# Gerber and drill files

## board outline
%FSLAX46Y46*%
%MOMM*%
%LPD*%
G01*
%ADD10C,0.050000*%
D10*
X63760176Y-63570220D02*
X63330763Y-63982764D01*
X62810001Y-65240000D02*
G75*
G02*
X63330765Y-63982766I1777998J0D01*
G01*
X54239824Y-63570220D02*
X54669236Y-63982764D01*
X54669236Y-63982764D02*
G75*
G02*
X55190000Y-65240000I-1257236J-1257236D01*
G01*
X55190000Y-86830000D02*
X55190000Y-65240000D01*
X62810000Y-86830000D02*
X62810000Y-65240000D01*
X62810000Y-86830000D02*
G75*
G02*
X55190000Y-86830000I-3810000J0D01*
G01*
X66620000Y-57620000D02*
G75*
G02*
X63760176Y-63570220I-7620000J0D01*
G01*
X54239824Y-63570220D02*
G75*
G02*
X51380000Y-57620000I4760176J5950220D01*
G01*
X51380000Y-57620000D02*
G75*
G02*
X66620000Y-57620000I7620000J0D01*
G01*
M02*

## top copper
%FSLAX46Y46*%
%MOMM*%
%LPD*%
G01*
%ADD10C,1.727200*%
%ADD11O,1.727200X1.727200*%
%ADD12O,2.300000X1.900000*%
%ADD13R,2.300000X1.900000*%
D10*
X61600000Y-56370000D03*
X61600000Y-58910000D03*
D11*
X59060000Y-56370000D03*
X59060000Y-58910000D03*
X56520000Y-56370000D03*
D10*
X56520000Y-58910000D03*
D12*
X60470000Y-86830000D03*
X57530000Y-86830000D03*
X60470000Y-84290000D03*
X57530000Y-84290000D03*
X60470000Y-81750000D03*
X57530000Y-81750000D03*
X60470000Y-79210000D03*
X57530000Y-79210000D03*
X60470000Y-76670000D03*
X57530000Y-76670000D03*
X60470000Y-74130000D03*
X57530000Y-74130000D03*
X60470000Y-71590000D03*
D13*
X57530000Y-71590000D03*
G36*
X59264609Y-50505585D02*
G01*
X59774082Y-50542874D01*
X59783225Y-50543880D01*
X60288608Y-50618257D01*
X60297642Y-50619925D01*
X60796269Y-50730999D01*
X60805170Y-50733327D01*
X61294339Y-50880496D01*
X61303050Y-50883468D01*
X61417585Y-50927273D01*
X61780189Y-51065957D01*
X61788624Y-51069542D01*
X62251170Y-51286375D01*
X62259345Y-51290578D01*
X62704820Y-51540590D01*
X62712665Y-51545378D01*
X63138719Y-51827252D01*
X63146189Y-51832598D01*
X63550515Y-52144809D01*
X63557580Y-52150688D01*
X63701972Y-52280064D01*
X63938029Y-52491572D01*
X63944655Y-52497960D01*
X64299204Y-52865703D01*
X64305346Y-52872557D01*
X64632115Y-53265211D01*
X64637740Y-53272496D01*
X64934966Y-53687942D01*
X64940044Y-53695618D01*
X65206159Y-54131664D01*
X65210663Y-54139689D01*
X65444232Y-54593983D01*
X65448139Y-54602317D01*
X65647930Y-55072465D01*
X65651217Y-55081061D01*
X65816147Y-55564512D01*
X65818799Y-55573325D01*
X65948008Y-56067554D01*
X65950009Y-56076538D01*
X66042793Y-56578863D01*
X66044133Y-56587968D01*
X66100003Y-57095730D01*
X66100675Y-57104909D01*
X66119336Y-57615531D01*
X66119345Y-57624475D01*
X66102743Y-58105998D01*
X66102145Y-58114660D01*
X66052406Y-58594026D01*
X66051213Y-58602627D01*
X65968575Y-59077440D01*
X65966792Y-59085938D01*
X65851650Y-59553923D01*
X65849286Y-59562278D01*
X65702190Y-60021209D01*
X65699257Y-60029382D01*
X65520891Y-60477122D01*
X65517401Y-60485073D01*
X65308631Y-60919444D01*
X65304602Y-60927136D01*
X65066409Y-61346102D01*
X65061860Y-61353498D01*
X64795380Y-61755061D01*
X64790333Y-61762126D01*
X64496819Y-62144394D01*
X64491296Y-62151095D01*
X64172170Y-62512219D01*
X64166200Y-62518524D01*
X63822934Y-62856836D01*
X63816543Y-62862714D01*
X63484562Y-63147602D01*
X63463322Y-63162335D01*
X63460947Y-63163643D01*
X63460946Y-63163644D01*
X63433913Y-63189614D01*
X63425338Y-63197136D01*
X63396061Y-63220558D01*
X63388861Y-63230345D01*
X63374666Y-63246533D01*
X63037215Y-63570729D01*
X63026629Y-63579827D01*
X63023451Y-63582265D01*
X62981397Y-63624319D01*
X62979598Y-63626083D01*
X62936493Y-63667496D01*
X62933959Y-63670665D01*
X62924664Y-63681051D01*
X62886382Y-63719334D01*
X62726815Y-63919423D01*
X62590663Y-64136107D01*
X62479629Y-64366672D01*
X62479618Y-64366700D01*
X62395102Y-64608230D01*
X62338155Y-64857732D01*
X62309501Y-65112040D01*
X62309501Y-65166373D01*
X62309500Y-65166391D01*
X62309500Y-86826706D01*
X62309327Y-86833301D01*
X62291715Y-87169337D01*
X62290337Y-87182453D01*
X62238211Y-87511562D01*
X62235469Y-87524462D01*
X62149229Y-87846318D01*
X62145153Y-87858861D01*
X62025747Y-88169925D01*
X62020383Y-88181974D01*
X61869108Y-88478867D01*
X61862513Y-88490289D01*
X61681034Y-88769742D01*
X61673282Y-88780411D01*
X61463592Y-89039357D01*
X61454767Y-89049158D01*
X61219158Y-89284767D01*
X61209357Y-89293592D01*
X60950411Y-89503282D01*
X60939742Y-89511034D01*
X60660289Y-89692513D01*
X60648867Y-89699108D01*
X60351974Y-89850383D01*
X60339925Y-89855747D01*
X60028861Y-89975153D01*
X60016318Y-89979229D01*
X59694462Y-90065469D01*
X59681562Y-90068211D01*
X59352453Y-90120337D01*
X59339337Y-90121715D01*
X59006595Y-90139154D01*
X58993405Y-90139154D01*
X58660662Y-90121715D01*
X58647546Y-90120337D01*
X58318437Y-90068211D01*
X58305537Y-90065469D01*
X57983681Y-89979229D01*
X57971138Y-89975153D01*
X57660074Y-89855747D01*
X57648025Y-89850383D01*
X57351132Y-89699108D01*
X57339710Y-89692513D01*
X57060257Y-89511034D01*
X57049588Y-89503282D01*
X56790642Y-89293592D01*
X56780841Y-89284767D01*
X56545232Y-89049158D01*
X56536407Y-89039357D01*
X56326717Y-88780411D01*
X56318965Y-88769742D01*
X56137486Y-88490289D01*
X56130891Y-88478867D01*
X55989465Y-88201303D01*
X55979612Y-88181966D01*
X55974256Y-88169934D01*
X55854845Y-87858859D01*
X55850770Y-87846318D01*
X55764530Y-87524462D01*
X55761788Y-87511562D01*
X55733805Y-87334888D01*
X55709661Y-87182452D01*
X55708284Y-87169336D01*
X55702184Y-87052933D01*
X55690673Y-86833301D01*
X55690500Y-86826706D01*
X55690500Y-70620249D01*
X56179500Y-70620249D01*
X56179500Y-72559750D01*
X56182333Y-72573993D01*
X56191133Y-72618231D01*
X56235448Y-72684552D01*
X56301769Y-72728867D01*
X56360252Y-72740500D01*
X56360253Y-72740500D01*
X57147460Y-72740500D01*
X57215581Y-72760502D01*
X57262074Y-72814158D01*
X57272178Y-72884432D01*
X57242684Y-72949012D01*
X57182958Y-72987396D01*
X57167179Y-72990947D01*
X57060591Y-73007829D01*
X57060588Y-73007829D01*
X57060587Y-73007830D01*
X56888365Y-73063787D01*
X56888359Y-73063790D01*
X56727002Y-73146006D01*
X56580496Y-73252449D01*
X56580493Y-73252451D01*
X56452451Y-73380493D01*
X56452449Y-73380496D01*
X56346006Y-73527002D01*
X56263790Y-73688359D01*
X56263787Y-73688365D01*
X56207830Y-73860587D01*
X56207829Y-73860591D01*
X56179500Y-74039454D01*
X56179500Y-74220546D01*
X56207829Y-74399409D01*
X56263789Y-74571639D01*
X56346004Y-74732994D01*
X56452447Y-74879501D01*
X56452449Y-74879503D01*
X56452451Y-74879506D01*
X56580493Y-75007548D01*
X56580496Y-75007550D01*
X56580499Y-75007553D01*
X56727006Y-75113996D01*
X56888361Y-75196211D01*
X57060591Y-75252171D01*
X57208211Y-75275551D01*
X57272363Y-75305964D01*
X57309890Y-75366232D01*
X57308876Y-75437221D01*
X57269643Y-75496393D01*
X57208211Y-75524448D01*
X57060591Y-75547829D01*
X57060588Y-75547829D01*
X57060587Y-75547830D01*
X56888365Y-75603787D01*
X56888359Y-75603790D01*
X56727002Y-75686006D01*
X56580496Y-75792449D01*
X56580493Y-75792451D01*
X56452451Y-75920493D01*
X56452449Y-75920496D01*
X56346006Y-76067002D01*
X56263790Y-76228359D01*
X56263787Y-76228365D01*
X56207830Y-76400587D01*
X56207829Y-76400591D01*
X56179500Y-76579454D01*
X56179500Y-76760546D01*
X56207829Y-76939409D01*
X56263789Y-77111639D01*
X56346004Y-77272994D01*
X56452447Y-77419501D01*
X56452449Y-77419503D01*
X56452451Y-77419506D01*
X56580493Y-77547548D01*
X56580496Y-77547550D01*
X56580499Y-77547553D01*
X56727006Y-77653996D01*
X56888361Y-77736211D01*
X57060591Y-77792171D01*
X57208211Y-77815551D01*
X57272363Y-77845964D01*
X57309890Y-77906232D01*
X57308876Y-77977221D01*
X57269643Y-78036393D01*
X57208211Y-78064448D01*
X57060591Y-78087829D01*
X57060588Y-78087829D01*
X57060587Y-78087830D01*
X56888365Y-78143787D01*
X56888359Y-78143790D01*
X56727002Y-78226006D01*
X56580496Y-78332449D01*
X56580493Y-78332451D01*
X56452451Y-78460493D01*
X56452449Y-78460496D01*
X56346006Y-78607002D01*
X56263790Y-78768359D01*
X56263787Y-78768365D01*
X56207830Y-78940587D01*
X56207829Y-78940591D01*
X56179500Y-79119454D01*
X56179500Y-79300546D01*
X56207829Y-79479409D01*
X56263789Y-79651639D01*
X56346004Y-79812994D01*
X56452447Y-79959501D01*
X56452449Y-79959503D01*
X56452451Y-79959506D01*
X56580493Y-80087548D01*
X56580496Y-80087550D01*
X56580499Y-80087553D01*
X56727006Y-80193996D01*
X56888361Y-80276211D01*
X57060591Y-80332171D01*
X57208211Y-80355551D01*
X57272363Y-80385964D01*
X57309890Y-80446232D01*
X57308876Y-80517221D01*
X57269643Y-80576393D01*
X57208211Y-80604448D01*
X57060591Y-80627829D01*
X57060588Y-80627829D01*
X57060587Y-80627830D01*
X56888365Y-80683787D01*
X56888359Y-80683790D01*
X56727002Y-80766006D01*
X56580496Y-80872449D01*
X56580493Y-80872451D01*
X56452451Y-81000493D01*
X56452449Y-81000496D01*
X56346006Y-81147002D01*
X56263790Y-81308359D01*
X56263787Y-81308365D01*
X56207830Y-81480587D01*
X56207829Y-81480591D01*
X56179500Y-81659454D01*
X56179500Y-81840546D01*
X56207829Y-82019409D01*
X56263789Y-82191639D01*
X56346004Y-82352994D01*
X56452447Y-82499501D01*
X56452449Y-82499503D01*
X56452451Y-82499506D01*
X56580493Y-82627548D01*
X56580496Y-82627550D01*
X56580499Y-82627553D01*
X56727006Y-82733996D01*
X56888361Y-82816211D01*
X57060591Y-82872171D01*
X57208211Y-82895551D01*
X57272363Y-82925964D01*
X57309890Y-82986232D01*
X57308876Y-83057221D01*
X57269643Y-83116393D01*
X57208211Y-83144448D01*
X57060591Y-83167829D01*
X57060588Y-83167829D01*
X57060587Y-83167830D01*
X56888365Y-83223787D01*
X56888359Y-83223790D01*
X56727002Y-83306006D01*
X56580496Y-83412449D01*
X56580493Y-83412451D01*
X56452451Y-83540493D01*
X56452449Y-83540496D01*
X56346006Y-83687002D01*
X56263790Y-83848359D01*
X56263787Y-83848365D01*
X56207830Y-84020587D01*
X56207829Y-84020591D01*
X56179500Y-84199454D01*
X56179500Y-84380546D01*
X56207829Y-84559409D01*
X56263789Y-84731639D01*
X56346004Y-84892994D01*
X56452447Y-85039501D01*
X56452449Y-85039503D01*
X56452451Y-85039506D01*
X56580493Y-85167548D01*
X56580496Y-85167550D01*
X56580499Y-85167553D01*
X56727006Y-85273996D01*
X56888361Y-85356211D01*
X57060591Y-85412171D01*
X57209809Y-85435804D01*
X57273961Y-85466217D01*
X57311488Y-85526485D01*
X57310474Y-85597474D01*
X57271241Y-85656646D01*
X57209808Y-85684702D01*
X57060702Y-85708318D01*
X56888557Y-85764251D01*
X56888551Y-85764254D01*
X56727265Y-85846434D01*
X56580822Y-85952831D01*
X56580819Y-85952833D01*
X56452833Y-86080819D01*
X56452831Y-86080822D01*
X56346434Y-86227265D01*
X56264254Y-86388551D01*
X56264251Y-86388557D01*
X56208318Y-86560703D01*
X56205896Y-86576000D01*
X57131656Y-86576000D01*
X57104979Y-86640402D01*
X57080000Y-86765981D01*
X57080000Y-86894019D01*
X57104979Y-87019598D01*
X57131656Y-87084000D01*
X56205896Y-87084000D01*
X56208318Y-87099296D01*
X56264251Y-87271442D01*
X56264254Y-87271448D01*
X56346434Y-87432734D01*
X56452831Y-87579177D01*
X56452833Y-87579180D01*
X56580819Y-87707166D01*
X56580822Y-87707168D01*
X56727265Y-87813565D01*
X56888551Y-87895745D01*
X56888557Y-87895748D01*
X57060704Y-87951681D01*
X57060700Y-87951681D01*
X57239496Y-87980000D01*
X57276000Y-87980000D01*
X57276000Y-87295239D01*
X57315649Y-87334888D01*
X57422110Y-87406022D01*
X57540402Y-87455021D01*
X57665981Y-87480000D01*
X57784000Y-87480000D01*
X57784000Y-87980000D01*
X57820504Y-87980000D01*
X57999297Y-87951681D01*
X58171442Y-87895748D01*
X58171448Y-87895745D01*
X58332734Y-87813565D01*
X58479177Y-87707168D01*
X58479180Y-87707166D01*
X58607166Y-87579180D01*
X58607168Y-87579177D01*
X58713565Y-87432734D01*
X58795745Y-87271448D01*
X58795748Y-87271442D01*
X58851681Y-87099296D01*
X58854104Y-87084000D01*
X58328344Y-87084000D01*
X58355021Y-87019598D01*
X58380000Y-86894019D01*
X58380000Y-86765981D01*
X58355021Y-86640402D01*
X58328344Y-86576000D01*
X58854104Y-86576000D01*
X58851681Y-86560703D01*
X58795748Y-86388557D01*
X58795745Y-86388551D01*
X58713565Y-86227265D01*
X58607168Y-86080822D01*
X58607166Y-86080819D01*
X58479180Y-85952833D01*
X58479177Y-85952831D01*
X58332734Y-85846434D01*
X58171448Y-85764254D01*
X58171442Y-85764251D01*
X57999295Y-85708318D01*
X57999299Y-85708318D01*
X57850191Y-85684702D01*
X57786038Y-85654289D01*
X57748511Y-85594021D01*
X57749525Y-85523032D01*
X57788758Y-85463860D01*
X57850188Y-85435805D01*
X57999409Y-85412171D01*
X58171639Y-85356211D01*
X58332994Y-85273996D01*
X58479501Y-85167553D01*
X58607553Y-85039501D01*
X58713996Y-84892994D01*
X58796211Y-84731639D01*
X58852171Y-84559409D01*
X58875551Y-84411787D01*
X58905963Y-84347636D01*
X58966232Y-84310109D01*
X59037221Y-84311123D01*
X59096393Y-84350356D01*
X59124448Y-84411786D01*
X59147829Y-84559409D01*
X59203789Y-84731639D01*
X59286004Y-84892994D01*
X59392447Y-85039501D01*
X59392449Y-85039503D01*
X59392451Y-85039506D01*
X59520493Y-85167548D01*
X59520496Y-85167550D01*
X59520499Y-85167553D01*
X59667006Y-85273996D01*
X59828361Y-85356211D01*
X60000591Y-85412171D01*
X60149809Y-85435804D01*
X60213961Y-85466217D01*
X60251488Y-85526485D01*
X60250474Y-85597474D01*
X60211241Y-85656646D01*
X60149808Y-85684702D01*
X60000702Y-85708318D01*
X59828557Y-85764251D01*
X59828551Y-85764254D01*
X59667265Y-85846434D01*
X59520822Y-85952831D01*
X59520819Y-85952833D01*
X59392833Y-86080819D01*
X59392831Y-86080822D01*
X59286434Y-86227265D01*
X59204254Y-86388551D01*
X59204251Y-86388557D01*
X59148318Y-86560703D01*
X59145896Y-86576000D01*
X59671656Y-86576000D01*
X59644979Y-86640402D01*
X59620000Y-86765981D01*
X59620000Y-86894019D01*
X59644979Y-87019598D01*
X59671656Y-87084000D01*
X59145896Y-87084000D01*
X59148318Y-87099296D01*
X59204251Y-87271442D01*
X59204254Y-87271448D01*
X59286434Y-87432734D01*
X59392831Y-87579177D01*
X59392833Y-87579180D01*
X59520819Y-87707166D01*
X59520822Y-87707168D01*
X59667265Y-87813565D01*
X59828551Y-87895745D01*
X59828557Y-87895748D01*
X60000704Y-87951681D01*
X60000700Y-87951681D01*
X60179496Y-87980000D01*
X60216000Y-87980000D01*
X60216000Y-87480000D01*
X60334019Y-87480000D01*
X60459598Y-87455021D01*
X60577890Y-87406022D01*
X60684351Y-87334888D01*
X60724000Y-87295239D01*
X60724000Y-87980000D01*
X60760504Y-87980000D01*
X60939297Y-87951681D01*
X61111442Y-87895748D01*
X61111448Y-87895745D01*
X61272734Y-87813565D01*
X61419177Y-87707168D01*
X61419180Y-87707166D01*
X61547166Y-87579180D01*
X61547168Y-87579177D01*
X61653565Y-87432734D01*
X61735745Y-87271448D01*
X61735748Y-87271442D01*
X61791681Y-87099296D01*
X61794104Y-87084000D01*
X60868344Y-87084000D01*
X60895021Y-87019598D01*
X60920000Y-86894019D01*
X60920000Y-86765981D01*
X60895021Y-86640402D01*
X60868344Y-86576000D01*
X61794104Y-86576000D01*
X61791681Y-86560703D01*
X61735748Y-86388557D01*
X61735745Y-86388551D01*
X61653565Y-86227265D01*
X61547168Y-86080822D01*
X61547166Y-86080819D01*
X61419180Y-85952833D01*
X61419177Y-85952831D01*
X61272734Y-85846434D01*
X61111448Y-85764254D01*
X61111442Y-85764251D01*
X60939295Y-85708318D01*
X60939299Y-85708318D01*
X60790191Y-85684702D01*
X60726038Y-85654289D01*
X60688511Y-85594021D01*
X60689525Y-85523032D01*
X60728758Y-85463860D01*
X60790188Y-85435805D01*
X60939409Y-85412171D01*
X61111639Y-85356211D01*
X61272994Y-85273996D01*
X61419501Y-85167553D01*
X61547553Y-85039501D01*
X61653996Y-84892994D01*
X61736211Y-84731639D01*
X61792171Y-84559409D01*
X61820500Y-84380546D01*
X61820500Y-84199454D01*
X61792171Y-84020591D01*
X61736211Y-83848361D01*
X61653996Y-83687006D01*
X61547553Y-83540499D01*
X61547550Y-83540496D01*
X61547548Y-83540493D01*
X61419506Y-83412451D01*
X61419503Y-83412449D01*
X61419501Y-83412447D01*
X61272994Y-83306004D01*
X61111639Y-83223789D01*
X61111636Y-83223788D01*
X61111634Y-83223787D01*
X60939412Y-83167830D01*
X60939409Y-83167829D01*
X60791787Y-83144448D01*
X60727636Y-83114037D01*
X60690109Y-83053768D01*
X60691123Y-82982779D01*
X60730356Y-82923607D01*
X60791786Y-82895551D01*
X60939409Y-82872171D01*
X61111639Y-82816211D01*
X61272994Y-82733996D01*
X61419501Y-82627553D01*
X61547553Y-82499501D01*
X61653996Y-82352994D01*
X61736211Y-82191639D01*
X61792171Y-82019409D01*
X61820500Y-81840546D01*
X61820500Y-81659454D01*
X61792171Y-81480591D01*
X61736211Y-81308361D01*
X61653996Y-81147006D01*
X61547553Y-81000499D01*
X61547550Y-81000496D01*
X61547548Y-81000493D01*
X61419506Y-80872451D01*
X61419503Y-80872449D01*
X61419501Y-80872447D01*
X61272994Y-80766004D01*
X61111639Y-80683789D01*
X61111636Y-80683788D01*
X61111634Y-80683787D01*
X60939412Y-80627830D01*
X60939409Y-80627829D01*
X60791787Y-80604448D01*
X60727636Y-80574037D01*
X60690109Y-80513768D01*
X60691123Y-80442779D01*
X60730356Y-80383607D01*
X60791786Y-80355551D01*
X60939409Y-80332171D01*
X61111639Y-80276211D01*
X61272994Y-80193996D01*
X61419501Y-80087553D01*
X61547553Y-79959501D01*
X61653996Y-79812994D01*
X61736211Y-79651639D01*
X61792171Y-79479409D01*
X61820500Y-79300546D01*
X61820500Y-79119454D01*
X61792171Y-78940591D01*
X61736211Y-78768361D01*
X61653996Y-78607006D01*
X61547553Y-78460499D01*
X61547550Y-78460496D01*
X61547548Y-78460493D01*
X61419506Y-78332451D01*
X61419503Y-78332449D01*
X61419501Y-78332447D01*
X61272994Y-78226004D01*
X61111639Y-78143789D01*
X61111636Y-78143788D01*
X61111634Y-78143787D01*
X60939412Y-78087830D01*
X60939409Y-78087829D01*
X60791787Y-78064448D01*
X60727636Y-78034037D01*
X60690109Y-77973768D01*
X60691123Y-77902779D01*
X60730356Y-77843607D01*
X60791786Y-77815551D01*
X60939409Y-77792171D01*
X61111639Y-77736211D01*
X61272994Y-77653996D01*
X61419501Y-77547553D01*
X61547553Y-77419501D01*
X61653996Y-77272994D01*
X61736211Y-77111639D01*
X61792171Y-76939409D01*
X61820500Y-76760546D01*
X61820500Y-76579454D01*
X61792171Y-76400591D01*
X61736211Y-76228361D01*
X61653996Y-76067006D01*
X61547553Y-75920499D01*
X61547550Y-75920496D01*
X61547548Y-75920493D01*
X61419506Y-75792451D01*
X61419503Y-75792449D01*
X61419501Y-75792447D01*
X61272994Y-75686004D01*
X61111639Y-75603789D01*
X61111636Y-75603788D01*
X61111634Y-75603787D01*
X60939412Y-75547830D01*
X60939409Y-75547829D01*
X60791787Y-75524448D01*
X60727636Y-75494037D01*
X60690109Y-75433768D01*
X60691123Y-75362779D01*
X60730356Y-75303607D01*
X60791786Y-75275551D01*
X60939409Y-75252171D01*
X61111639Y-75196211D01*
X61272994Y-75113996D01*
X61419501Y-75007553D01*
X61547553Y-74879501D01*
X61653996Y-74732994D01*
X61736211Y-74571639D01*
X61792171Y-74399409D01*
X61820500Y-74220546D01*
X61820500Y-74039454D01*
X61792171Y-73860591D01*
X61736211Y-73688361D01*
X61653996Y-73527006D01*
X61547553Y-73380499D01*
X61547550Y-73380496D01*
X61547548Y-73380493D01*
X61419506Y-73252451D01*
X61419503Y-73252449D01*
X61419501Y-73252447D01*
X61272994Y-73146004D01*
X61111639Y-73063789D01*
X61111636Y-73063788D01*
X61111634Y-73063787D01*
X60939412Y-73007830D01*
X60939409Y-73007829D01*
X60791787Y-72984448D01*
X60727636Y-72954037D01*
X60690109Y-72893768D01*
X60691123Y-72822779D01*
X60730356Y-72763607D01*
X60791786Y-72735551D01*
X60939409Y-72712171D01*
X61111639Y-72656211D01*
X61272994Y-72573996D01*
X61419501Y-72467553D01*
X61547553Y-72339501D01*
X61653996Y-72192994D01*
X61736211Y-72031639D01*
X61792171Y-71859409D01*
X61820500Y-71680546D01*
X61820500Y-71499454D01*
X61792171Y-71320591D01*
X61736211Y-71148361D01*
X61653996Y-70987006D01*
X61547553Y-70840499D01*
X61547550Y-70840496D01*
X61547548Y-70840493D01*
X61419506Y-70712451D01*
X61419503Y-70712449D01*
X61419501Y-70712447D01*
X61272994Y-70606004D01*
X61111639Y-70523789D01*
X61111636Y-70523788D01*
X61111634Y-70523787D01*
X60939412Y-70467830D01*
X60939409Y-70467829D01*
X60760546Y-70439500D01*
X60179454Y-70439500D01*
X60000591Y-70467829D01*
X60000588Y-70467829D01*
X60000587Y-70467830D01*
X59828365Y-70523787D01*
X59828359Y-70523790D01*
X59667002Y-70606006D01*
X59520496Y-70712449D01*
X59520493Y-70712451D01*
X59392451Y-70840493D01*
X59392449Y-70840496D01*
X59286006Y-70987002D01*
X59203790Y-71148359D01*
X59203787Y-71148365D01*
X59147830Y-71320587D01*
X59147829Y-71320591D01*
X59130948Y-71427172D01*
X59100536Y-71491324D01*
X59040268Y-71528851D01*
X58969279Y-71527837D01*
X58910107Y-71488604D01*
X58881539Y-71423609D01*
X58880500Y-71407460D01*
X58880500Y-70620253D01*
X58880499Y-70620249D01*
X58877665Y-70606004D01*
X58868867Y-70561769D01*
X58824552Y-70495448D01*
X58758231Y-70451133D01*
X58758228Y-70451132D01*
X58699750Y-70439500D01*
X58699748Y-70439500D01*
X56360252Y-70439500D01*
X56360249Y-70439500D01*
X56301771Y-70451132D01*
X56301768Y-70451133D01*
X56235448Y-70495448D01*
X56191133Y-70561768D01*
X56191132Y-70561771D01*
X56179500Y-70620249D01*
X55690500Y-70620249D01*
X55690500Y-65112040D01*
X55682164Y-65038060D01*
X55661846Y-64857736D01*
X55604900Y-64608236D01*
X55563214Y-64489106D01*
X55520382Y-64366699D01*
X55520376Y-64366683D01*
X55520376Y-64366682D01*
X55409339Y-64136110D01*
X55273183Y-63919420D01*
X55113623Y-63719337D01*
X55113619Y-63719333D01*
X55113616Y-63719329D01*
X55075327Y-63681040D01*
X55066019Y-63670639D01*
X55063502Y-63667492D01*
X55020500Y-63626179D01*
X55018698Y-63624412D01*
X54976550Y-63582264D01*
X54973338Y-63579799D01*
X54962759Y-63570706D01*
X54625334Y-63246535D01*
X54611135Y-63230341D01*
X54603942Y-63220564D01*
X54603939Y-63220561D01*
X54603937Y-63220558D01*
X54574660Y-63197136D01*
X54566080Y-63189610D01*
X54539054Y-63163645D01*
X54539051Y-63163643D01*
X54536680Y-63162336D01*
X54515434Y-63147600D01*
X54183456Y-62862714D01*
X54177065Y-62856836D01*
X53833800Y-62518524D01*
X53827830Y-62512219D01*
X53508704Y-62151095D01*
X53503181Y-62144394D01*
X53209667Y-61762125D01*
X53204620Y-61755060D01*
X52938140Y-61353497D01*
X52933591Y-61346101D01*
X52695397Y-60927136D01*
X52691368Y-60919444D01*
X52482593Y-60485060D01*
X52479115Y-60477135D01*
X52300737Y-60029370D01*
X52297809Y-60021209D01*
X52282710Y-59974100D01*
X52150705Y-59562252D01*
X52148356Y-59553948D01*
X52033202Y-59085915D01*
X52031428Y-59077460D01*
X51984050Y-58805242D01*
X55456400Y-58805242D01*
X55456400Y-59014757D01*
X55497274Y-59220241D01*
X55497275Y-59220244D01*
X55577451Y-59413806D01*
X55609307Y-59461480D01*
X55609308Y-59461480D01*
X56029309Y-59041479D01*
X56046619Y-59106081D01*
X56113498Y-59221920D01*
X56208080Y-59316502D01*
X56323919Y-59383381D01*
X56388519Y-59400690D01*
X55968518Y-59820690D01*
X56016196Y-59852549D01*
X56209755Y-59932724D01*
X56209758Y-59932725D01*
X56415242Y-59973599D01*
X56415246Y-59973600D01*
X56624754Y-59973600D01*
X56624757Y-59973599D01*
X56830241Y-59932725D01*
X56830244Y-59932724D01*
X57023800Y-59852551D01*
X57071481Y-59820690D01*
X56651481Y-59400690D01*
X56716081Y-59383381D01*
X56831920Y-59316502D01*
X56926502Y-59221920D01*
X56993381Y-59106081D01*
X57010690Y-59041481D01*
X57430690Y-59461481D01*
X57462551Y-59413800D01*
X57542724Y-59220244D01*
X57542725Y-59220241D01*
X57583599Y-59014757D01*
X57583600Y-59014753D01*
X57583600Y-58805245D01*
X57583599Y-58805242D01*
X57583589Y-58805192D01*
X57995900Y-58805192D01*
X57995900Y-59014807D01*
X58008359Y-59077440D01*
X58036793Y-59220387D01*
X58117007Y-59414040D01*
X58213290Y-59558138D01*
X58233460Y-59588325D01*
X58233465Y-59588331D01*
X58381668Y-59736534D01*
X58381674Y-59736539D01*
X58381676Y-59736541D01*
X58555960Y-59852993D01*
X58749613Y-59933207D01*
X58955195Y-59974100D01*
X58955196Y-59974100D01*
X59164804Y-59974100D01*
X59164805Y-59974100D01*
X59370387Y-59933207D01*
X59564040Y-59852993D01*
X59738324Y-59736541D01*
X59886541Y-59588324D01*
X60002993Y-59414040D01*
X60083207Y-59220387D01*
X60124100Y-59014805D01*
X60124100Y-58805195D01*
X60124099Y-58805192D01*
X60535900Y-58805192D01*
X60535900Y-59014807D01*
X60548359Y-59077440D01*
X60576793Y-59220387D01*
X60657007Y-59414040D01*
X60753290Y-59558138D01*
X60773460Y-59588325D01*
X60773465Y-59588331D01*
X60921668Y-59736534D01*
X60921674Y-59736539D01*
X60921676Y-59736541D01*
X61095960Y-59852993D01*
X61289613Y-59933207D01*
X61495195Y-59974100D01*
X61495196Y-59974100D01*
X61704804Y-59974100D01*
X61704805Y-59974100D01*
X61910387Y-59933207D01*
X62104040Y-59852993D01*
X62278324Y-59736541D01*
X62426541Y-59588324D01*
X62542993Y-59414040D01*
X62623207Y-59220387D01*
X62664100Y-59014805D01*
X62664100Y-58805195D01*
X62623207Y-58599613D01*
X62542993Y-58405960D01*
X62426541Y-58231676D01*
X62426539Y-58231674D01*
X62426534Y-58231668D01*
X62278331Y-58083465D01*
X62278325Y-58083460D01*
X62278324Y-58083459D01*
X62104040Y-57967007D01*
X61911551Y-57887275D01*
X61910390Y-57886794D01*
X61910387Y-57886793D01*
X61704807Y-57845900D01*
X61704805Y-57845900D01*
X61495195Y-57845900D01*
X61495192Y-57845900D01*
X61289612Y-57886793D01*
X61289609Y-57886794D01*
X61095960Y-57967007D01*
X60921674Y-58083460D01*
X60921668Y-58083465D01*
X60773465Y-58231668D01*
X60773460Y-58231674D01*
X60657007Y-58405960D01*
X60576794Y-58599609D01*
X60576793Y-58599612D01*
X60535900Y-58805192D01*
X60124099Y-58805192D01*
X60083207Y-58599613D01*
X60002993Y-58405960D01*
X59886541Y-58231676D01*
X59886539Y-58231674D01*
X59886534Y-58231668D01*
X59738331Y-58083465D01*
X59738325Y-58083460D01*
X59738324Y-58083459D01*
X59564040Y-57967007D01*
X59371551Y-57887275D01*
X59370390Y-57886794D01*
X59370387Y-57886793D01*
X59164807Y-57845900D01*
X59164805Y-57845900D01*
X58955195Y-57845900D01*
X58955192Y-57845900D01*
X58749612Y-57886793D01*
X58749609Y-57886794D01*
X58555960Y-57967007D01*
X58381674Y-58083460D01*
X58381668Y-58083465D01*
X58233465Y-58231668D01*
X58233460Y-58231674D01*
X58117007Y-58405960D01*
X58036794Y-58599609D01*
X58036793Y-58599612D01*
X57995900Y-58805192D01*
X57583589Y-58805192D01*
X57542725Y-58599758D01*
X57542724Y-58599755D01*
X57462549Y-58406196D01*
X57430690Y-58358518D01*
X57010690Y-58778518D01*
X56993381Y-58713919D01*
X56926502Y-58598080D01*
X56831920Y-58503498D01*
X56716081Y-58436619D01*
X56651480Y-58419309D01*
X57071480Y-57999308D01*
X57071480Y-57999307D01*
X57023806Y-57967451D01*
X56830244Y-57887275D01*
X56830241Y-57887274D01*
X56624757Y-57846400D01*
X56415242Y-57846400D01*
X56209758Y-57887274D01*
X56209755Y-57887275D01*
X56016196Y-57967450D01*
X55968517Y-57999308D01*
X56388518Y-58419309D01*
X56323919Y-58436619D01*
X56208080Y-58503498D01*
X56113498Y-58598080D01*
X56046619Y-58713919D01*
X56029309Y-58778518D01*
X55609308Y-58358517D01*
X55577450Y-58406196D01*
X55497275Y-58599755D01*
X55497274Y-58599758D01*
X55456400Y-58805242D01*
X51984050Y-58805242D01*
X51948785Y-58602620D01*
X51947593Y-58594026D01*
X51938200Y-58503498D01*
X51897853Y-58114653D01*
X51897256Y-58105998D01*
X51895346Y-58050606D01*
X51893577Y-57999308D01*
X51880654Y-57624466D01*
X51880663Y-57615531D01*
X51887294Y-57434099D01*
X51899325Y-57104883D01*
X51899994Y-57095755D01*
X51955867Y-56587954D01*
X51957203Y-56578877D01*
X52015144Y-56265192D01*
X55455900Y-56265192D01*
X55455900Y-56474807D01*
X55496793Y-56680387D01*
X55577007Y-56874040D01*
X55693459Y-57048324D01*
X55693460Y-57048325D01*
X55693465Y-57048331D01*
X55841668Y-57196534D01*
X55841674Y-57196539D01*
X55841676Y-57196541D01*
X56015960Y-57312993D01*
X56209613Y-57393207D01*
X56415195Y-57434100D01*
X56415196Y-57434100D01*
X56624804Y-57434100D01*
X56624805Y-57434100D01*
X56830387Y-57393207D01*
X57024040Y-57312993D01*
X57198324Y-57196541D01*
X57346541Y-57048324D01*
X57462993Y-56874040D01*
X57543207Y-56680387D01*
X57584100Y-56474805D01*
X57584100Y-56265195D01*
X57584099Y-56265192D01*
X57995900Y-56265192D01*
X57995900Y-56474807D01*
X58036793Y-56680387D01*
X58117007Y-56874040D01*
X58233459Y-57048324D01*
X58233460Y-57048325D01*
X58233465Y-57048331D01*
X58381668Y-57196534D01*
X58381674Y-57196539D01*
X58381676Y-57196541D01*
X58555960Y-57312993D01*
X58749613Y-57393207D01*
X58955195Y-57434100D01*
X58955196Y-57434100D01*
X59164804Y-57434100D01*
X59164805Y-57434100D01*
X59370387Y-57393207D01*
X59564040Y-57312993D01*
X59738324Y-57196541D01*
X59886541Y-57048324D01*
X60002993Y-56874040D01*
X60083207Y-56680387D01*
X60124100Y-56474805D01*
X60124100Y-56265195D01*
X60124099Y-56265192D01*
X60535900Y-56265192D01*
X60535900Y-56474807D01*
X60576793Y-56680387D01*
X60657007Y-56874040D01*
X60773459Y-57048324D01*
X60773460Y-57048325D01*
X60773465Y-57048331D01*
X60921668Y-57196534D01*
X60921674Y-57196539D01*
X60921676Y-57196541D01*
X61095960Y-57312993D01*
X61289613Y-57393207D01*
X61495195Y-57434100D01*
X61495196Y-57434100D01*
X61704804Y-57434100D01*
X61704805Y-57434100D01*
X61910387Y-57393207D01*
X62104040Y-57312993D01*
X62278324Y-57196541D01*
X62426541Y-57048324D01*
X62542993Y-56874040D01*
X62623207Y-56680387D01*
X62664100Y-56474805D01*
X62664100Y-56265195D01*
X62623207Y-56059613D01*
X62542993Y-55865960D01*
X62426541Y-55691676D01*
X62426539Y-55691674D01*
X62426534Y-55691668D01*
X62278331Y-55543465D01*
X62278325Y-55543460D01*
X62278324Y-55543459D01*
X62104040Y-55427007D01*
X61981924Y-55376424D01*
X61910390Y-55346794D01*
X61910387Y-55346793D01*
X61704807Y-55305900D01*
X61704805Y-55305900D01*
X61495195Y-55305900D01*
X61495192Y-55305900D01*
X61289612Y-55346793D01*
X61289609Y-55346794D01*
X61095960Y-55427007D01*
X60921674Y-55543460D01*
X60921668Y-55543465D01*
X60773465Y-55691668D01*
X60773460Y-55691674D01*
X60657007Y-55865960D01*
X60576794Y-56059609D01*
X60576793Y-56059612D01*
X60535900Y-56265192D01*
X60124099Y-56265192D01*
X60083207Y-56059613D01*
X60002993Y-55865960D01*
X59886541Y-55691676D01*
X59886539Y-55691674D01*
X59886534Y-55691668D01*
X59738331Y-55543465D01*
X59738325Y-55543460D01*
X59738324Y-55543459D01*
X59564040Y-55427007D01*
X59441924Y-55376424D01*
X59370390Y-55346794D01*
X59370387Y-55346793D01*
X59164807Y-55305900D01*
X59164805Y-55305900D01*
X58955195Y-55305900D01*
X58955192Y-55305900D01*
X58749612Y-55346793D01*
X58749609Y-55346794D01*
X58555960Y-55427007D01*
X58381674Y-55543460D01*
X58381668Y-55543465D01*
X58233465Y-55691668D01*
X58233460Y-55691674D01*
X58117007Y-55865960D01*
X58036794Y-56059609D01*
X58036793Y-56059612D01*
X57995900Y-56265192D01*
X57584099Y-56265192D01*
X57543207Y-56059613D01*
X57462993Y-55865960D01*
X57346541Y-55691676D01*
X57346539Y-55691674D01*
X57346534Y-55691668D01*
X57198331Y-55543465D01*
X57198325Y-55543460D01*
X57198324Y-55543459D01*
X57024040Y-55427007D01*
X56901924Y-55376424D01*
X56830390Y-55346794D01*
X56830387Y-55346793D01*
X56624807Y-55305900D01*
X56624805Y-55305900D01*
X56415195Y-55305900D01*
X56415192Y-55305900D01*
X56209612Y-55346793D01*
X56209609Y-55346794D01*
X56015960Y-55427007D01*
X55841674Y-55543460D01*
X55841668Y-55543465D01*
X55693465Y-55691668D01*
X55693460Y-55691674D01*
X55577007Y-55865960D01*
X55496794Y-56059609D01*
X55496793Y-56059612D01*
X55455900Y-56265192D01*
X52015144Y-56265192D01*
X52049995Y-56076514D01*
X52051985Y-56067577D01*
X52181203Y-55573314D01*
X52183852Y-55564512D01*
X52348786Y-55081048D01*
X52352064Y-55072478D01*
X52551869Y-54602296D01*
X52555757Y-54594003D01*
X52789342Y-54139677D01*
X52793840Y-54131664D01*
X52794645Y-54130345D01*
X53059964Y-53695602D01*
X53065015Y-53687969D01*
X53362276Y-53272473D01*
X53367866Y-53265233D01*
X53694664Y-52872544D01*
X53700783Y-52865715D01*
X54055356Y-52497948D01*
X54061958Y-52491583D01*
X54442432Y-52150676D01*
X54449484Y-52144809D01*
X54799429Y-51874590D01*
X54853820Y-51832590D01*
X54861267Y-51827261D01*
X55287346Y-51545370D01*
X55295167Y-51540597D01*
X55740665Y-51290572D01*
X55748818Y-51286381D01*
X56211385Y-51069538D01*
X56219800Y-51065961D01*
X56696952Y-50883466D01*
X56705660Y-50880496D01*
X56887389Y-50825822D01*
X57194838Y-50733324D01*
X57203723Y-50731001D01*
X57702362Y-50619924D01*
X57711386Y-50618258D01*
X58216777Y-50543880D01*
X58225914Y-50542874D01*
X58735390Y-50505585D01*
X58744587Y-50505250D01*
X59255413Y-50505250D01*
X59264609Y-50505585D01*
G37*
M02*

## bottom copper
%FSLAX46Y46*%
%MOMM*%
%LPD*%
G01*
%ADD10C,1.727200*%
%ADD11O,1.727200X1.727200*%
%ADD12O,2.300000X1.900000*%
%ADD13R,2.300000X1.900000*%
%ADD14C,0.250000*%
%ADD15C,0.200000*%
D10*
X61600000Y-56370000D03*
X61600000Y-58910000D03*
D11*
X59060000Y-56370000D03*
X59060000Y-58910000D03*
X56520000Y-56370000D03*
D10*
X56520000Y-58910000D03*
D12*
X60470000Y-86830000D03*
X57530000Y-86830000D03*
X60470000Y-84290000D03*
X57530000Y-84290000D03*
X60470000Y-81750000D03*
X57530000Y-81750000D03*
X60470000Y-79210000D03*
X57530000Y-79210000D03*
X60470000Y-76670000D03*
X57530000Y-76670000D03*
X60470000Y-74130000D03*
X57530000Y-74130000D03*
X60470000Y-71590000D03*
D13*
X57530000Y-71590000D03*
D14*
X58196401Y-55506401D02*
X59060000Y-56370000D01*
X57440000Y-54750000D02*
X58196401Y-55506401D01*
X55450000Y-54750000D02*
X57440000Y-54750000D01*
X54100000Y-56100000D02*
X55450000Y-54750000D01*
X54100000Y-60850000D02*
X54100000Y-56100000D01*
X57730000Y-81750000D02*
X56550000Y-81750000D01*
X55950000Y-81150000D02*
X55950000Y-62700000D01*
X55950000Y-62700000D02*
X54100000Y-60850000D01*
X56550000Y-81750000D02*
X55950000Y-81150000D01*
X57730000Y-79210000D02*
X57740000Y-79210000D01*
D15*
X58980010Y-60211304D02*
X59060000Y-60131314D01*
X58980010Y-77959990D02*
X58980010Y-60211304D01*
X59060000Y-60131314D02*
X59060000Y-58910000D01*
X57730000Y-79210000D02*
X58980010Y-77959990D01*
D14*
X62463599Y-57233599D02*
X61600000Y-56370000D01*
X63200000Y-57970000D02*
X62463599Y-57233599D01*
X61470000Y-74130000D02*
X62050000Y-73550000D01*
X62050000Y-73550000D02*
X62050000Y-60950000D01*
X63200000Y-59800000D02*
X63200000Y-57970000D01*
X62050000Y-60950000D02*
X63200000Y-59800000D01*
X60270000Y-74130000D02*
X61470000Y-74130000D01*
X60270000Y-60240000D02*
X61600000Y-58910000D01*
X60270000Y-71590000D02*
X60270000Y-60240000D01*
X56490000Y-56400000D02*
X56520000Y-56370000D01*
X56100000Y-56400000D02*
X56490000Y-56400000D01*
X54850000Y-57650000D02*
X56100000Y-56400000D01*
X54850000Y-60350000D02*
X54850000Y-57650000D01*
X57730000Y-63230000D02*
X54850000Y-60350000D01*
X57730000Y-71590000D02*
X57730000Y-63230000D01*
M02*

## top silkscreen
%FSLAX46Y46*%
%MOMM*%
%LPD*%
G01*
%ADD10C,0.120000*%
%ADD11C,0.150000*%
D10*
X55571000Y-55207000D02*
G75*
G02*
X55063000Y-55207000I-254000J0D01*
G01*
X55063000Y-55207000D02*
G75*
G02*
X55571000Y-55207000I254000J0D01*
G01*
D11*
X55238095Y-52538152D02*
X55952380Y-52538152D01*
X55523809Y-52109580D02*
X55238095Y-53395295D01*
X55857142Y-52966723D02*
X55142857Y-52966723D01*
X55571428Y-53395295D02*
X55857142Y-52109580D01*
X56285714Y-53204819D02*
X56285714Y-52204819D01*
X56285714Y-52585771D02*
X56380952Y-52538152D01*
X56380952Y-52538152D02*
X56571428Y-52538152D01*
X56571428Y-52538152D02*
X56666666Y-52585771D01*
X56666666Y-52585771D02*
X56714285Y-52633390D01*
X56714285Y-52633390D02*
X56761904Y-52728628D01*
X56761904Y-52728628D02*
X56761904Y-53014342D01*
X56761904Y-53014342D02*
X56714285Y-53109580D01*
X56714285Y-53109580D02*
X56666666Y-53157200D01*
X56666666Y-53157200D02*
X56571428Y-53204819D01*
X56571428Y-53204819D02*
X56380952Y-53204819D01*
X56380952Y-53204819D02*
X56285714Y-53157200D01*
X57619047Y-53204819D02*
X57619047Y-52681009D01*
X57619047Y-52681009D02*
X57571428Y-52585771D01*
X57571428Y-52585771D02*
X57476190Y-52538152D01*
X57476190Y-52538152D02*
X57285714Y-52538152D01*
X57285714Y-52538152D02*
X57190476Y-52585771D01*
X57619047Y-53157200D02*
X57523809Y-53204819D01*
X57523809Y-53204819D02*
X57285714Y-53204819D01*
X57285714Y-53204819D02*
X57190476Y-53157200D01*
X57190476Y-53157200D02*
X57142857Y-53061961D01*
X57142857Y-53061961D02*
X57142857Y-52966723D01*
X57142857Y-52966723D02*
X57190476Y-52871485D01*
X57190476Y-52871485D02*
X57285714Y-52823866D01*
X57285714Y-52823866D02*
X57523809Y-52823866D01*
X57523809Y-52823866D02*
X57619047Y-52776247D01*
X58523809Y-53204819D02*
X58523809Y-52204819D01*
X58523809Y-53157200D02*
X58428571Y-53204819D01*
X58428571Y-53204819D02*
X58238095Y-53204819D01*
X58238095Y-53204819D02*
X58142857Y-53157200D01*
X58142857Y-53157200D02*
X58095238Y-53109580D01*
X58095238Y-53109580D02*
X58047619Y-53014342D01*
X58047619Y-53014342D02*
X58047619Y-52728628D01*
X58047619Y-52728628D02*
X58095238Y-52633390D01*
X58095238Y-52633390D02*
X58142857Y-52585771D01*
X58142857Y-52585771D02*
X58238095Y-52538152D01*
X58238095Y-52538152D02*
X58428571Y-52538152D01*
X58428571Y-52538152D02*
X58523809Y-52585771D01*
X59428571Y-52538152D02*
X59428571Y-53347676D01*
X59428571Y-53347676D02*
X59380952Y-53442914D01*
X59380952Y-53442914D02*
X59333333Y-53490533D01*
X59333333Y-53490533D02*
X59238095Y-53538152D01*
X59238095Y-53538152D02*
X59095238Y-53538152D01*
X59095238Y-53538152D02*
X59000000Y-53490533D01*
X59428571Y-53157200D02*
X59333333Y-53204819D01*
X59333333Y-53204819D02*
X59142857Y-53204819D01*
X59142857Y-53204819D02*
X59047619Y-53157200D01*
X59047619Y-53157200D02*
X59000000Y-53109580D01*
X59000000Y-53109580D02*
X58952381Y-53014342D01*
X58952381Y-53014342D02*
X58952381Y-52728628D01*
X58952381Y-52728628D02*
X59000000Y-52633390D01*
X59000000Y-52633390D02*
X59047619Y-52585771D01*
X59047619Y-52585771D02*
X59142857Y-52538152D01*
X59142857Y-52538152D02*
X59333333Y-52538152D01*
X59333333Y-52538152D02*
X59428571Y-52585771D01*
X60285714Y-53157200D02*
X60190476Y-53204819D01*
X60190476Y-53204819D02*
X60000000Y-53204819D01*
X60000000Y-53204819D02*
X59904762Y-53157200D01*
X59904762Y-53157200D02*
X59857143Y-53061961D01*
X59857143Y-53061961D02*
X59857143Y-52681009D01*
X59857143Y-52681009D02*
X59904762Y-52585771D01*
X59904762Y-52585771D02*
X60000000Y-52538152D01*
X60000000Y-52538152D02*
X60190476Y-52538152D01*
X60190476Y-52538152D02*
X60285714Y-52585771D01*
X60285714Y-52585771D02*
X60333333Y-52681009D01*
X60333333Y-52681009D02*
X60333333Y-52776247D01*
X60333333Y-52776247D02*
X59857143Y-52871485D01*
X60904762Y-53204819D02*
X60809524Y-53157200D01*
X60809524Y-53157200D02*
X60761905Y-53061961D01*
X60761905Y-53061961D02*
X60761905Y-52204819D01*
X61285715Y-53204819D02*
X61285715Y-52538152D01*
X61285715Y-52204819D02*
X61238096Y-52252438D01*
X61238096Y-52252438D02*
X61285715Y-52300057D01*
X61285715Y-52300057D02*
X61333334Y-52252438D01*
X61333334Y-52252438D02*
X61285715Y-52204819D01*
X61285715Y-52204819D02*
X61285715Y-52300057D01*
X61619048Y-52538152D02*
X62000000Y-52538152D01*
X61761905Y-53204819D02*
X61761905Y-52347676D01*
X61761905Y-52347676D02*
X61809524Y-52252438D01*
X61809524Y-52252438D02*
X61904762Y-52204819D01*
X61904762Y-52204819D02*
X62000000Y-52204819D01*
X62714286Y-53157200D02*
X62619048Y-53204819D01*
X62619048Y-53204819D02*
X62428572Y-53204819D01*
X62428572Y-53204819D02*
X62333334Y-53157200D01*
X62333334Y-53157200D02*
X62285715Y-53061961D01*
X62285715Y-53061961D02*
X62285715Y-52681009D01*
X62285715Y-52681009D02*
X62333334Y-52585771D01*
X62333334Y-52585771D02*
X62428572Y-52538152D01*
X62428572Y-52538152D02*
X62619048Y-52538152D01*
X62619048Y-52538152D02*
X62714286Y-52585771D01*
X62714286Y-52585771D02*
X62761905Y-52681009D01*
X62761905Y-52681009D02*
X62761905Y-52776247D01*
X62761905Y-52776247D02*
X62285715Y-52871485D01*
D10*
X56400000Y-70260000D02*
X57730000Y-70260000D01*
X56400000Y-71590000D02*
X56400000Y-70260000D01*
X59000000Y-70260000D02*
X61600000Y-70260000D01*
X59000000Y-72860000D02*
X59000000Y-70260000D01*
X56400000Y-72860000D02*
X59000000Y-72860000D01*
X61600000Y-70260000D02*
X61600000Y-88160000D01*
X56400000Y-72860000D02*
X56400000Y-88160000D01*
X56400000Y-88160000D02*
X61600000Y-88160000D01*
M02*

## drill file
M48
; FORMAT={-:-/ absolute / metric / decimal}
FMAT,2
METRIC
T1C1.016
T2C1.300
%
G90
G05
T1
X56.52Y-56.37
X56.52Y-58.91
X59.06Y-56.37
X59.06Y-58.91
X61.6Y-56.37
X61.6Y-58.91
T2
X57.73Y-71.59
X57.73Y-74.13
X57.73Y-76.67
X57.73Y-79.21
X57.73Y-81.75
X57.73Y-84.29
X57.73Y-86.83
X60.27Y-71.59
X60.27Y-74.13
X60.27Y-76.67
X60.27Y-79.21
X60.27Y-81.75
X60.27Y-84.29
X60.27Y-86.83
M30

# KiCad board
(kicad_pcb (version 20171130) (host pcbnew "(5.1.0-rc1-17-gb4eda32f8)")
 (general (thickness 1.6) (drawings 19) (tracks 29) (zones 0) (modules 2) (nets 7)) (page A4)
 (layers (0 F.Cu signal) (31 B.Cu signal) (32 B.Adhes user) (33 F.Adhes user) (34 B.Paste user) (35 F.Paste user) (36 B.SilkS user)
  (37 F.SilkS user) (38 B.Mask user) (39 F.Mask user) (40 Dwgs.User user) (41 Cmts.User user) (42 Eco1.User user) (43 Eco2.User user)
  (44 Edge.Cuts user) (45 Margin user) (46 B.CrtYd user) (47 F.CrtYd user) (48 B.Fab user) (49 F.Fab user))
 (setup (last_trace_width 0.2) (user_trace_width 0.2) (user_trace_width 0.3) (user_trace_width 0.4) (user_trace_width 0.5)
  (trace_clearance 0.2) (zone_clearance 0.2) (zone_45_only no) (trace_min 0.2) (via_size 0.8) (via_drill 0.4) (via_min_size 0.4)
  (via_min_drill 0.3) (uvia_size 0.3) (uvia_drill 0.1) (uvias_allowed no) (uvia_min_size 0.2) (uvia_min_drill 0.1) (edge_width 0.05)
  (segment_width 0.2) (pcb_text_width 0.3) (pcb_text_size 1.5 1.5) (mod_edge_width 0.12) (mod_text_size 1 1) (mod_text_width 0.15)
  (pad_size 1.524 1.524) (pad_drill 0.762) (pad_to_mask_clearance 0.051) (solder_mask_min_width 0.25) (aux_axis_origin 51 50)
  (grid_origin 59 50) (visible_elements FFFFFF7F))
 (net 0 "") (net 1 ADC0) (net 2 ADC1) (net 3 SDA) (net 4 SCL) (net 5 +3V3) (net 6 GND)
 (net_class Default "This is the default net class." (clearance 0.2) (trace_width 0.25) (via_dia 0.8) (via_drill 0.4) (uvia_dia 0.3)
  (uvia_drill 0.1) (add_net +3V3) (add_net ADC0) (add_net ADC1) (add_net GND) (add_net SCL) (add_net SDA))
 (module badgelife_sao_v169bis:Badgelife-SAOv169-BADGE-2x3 (layer F.Cu) (at 59 57.62)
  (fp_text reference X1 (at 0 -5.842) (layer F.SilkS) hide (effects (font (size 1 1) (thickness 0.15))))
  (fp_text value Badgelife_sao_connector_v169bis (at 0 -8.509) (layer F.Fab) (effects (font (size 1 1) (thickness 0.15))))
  (pad 5 thru_hole circle (at 2.6 -1.25 270) (size 1.7272 1.7272) (drill 1.016) (layers *.Cu *.Mask) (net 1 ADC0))
  (pad 6 thru_hole circle (at 2.6 1.29 270) (size 1.7272 1.7272) (drill 1.016) (layers *.Cu *.Mask) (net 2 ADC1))
  (pad 3 thru_hole oval (at 0.06 -1.25 270) (size 1.7272 1.7272) (drill 1.016) (layers *.Cu *.Mask) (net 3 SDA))
  (pad 4 thru_hole oval (at 0.06 1.29 270) (size 1.7272 1.7272) (drill 1.016) (layers *.Cu *.Mask) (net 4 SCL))
  (pad 1 thru_hole oval (at -2.48 -1.25 270) (size 1.7272 1.7272) (drill 1.016) (layers *.Cu *.Mask) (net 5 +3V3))
  (pad 2 thru_hole circle (at -2.48 1.29 270) (size 1.7272 1.7272) (drill 1.016) (layers *.Cu *.Mask) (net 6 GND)))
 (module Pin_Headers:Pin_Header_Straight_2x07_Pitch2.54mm (layer F.Cu) (at 57.73 71.59)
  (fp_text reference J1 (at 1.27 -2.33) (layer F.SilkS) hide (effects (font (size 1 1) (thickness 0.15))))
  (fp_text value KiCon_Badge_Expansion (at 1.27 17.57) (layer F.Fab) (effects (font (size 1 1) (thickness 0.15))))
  (fp_line (start -1.33 -1.33) (end 0 -1.33) (layer F.SilkS) (width 0.12))
  (fp_line (start -1.33 0) (end -1.33 -1.33) (layer F.SilkS) (width 0.12))
  (fp_line (start 1.27 -1.33) (end 3.87 -1.33) (layer F.SilkS) (width 0.12))
  (fp_line (start 1.27 1.27) (end 1.27 -1.33) (layer F.SilkS) (width 0.12))
  (fp_line (start -1.33 1.27) (end 1.27 1.27) (layer F.SilkS) (width 0.12))
  (fp_line (start 3.87 -1.33) (end 3.87 16.57) (layer F.SilkS) (width 0.12))
  (fp_line (start -1.33 1.27) (end -1.33 16.57) (layer F.SilkS) (width 0.12))
  (fp_line (start -1.33 16.57) (end 3.87 16.57) (layer F.SilkS) (width 0.12))
  (pad 14 thru_hole oval (at 2.54 15.24) (size 2.3 1.9) (drill 1.3 (offset 0.2 0)) (layers *.Cu *.Mask) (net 6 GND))
  (pad 13 thru_hole oval (at 0 15.24) (size 2.3 1.9) (drill 1.3 (offset -0.2 0)) (layers *.Cu *.Mask) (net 6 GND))
  (pad 12 thru_hole oval (at 2.54 12.7) (size 2.3 1.9) (drill 1.3 (offset 0.2 0)) (layers *.Cu *.Mask))
  (pad 11 thru_hole oval (at 0 12.7) (size 2.3 1.9) (drill 1.3 (offset -0.2 0)) (layers *.Cu *.Mask))
  (pad 10 thru_hole oval (at 2.54 10.16) (size 2.3 1.9) (drill 1.3 (offset 0.2 0)) (layers *.Cu *.Mask))
  (pad 9 thru_hole oval (at 0 10.16) (size 2.3 1.9) (drill 1.3 (offset -0.2 0)) (layers *.Cu *.Mask) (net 3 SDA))
  (pad 8 thru_hole oval (at 2.54 7.62) (size 2.3 1.9) (drill 1.3 (offset 0.2 0)) (layers *.Cu *.Mask))
  (pad 7 thru_hole oval (at 0 7.62) (size 2.3 1.9) (drill 1.3 (offset -0.2 0)) (layers *.Cu *.Mask) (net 4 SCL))
  (pad 6 thru_hole oval (at 2.54 5.08) (size 2.3 1.9) (drill 1.3 (offset 0.2 0)) (layers *.Cu *.Mask))
  (pad 5 thru_hole oval (at 0 5.08) (size 2.3 1.9) (drill 1.3 (offset -0.2 0)) (layers *.Cu *.Mask))
  (pad 4 thru_hole oval (at 2.54 2.54) (size 2.3 1.9) (drill 1.3 (offset 0.2 0)) (layers *.Cu *.Mask) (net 1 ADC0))
  (pad 3 thru_hole oval (at 0 2.54) (size 2.3 1.9) (drill 1.3 (offset -0.2 0)) (layers *.Cu *.Mask))
  (pad 2 thru_hole oval (at 2.54 0) (size 2.3 1.9) (drill 1.3 (offset 0.2 0)) (layers *.Cu *.Mask) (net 2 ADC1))
  (pad 1 thru_hole rect (at 0 0) (size 2.3 1.9) (drill 1.3 (offset -0.2 0)) (layers *.Cu *.Mask) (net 5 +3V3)))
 (gr_arc (start 55.317 55.207) (end 55.063 55.207) (angle -180) (layer F.SilkS) (width 0.12))
 (gr_arc (start 55.317 55.207) (end 55.571 55.207) (angle -180) (layer F.SilkS) (width 0.12))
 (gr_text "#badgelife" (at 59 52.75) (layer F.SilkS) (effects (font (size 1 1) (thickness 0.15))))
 (gr_line (start 63.760176 63.57022) (end 63.330763 63.982764) (layer Edge.Cuts) (width 0.05))
 (gr_arc (start 64.587999 65.24) (end 62.810001 65.24) (angle 45) (layer Edge.Cuts) (width 0.05))
 (gr_line (start 54.239824 63.57022) (end 54.669236 63.982764) (layer Edge.Cuts) (width 0.05))
 (gr_arc (start 53.412 65.24) (end 55.19 65.24) (angle -45) (layer Edge.Cuts) (width 0.05))
 (gr_line (start 55.19 86.83) (end 55.19 65.24) (layer Edge.Cuts) (width 0.05))
 (gr_line (start 62.81 86.83) (end 62.81 65.24) (layer Edge.Cuts) (width 0.05))
 (gr_arc (start 59 86.83) (end 55.19 86.83) (angle -180) (layer Edge.Cuts) (width 0.05))
 (gr_arc (start 59 57.62) (end 66.62 57.62) (angle 51.34019175) (layer Edge.Cuts) (width 0.05))
 (gr_arc (start 59 57.62) (end 51.38 57.62) (angle -51.34019175) (layer Edge.Cuts) (width 0.05))
 (gr_arc (start 59 57.62) (end 66.62 57.62) (angle -180) (layer Edge.Cuts) (width 0.05))
 (segment (start 58.196401 55.506401) (end 59.06 56.37) (width 0.25) (layer B.Cu) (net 3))
 (segment (start 57.44 54.75) (end 58.196401 55.506401) (width 0.25) (layer B.Cu) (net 3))
 (segment (start 55.45 54.75) (end 57.44 54.75) (width 0.25) (layer B.Cu) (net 3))
 (segment (start 54.1 56.1) (end 55.45 54.75) (width 0.25) (layer B.Cu) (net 3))
 (segment (start 54.1 60.85) (end 54.1 56.1) (width 0.25) (layer B.Cu) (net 3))
 (segment (start 57.73 81.75) (end 56.55 81.75) (width 0.25) (layer B.Cu) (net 3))
 (segment (start 55.95 81.15) (end 55.95 62.7) (width 0.25) (layer B.Cu) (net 3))
 (segment (start 55.95 62.7) (end 54.1 60.85) (width 0.25) (layer B.Cu) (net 3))
 (segment (start 56.55 81.75) (end 55.95 81.15) (width 0.25) (layer B.Cu) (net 3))
 (segment (start 57.73 79.21) (end 57.74 79.21) (width 0.25) (layer B.Cu) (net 4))
 (segment (start 58.98001 60.211304) (end 59.06 60.131314) (width 0.2) (layer B.Cu) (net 4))
 (segment (start 58.98001 77.95999) (end 58.98001 60.211304) (width 0.2) (layer B.Cu) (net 4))
 (segment (start 59.06 60.131314) (end 59.06 58.91) (width 0.2) (layer B.Cu) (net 4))
 (segment (start 57.73 79.21) (end 58.98001 77.95999) (width 0.2) (layer B.Cu) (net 4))
 (segment (start 62.463599 57.233599) (end 61.6 56.37) (width 0.25) (layer B.Cu) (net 1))
 (segment (start 63.2 57.97) (end 62.463599 57.233599) (width 0.25) (layer B.Cu) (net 1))
 (segment (start 61.47 74.13) (end 62.05 73.55) (width 0.25) (layer B.Cu) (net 1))
 (segment (start 62.05 73.55) (end 62.05 60.95) (width 0.25) (layer B.Cu) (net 1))
 (segment (start 63.2 59.8) (end 63.2 57.97) (width 0.25) (layer B.Cu) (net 1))
 (segment (start 62.05 60.95) (end 63.2 59.8) (width 0.25) (layer B.Cu) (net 1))
 (segment (start 60.27 74.13) (end 61.47 74.13) (width 0.25) (layer B.Cu) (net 1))
 (segment (start 60.27 60.24) (end 61.6 58.91) (width 0.25) (layer B.Cu) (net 2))
 (segment (start 60.27 71.59) (end 60.27 60.24) (width 0.25) (layer B.Cu) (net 2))
 (segment (start 56.49 56.4) (end 56.52 56.37) (width 0.25) (layer B.Cu) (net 5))
 (segment (start 56.1 56.4) (end 56.49 56.4) (width 0.25) (layer B.Cu) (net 5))
 (segment (start 54.85 57.65) (end 56.1 56.4) (width 0.25) (layer B.Cu) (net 5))
 (segment (start 54.85 60.35) (end 54.85 57.65) (width 0.25) (layer B.Cu) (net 5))
 (segment (start 57.73 63.23) (end 54.85 60.35) (width 0.25) (layer B.Cu) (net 5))
 (segment (start 57.73 71.59) (end 57.73 63.23) (width 0.25) (layer B.Cu) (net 5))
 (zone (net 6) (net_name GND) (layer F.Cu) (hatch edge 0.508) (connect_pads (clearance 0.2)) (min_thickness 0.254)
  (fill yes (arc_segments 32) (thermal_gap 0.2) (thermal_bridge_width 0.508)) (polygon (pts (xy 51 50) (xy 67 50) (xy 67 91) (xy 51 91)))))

